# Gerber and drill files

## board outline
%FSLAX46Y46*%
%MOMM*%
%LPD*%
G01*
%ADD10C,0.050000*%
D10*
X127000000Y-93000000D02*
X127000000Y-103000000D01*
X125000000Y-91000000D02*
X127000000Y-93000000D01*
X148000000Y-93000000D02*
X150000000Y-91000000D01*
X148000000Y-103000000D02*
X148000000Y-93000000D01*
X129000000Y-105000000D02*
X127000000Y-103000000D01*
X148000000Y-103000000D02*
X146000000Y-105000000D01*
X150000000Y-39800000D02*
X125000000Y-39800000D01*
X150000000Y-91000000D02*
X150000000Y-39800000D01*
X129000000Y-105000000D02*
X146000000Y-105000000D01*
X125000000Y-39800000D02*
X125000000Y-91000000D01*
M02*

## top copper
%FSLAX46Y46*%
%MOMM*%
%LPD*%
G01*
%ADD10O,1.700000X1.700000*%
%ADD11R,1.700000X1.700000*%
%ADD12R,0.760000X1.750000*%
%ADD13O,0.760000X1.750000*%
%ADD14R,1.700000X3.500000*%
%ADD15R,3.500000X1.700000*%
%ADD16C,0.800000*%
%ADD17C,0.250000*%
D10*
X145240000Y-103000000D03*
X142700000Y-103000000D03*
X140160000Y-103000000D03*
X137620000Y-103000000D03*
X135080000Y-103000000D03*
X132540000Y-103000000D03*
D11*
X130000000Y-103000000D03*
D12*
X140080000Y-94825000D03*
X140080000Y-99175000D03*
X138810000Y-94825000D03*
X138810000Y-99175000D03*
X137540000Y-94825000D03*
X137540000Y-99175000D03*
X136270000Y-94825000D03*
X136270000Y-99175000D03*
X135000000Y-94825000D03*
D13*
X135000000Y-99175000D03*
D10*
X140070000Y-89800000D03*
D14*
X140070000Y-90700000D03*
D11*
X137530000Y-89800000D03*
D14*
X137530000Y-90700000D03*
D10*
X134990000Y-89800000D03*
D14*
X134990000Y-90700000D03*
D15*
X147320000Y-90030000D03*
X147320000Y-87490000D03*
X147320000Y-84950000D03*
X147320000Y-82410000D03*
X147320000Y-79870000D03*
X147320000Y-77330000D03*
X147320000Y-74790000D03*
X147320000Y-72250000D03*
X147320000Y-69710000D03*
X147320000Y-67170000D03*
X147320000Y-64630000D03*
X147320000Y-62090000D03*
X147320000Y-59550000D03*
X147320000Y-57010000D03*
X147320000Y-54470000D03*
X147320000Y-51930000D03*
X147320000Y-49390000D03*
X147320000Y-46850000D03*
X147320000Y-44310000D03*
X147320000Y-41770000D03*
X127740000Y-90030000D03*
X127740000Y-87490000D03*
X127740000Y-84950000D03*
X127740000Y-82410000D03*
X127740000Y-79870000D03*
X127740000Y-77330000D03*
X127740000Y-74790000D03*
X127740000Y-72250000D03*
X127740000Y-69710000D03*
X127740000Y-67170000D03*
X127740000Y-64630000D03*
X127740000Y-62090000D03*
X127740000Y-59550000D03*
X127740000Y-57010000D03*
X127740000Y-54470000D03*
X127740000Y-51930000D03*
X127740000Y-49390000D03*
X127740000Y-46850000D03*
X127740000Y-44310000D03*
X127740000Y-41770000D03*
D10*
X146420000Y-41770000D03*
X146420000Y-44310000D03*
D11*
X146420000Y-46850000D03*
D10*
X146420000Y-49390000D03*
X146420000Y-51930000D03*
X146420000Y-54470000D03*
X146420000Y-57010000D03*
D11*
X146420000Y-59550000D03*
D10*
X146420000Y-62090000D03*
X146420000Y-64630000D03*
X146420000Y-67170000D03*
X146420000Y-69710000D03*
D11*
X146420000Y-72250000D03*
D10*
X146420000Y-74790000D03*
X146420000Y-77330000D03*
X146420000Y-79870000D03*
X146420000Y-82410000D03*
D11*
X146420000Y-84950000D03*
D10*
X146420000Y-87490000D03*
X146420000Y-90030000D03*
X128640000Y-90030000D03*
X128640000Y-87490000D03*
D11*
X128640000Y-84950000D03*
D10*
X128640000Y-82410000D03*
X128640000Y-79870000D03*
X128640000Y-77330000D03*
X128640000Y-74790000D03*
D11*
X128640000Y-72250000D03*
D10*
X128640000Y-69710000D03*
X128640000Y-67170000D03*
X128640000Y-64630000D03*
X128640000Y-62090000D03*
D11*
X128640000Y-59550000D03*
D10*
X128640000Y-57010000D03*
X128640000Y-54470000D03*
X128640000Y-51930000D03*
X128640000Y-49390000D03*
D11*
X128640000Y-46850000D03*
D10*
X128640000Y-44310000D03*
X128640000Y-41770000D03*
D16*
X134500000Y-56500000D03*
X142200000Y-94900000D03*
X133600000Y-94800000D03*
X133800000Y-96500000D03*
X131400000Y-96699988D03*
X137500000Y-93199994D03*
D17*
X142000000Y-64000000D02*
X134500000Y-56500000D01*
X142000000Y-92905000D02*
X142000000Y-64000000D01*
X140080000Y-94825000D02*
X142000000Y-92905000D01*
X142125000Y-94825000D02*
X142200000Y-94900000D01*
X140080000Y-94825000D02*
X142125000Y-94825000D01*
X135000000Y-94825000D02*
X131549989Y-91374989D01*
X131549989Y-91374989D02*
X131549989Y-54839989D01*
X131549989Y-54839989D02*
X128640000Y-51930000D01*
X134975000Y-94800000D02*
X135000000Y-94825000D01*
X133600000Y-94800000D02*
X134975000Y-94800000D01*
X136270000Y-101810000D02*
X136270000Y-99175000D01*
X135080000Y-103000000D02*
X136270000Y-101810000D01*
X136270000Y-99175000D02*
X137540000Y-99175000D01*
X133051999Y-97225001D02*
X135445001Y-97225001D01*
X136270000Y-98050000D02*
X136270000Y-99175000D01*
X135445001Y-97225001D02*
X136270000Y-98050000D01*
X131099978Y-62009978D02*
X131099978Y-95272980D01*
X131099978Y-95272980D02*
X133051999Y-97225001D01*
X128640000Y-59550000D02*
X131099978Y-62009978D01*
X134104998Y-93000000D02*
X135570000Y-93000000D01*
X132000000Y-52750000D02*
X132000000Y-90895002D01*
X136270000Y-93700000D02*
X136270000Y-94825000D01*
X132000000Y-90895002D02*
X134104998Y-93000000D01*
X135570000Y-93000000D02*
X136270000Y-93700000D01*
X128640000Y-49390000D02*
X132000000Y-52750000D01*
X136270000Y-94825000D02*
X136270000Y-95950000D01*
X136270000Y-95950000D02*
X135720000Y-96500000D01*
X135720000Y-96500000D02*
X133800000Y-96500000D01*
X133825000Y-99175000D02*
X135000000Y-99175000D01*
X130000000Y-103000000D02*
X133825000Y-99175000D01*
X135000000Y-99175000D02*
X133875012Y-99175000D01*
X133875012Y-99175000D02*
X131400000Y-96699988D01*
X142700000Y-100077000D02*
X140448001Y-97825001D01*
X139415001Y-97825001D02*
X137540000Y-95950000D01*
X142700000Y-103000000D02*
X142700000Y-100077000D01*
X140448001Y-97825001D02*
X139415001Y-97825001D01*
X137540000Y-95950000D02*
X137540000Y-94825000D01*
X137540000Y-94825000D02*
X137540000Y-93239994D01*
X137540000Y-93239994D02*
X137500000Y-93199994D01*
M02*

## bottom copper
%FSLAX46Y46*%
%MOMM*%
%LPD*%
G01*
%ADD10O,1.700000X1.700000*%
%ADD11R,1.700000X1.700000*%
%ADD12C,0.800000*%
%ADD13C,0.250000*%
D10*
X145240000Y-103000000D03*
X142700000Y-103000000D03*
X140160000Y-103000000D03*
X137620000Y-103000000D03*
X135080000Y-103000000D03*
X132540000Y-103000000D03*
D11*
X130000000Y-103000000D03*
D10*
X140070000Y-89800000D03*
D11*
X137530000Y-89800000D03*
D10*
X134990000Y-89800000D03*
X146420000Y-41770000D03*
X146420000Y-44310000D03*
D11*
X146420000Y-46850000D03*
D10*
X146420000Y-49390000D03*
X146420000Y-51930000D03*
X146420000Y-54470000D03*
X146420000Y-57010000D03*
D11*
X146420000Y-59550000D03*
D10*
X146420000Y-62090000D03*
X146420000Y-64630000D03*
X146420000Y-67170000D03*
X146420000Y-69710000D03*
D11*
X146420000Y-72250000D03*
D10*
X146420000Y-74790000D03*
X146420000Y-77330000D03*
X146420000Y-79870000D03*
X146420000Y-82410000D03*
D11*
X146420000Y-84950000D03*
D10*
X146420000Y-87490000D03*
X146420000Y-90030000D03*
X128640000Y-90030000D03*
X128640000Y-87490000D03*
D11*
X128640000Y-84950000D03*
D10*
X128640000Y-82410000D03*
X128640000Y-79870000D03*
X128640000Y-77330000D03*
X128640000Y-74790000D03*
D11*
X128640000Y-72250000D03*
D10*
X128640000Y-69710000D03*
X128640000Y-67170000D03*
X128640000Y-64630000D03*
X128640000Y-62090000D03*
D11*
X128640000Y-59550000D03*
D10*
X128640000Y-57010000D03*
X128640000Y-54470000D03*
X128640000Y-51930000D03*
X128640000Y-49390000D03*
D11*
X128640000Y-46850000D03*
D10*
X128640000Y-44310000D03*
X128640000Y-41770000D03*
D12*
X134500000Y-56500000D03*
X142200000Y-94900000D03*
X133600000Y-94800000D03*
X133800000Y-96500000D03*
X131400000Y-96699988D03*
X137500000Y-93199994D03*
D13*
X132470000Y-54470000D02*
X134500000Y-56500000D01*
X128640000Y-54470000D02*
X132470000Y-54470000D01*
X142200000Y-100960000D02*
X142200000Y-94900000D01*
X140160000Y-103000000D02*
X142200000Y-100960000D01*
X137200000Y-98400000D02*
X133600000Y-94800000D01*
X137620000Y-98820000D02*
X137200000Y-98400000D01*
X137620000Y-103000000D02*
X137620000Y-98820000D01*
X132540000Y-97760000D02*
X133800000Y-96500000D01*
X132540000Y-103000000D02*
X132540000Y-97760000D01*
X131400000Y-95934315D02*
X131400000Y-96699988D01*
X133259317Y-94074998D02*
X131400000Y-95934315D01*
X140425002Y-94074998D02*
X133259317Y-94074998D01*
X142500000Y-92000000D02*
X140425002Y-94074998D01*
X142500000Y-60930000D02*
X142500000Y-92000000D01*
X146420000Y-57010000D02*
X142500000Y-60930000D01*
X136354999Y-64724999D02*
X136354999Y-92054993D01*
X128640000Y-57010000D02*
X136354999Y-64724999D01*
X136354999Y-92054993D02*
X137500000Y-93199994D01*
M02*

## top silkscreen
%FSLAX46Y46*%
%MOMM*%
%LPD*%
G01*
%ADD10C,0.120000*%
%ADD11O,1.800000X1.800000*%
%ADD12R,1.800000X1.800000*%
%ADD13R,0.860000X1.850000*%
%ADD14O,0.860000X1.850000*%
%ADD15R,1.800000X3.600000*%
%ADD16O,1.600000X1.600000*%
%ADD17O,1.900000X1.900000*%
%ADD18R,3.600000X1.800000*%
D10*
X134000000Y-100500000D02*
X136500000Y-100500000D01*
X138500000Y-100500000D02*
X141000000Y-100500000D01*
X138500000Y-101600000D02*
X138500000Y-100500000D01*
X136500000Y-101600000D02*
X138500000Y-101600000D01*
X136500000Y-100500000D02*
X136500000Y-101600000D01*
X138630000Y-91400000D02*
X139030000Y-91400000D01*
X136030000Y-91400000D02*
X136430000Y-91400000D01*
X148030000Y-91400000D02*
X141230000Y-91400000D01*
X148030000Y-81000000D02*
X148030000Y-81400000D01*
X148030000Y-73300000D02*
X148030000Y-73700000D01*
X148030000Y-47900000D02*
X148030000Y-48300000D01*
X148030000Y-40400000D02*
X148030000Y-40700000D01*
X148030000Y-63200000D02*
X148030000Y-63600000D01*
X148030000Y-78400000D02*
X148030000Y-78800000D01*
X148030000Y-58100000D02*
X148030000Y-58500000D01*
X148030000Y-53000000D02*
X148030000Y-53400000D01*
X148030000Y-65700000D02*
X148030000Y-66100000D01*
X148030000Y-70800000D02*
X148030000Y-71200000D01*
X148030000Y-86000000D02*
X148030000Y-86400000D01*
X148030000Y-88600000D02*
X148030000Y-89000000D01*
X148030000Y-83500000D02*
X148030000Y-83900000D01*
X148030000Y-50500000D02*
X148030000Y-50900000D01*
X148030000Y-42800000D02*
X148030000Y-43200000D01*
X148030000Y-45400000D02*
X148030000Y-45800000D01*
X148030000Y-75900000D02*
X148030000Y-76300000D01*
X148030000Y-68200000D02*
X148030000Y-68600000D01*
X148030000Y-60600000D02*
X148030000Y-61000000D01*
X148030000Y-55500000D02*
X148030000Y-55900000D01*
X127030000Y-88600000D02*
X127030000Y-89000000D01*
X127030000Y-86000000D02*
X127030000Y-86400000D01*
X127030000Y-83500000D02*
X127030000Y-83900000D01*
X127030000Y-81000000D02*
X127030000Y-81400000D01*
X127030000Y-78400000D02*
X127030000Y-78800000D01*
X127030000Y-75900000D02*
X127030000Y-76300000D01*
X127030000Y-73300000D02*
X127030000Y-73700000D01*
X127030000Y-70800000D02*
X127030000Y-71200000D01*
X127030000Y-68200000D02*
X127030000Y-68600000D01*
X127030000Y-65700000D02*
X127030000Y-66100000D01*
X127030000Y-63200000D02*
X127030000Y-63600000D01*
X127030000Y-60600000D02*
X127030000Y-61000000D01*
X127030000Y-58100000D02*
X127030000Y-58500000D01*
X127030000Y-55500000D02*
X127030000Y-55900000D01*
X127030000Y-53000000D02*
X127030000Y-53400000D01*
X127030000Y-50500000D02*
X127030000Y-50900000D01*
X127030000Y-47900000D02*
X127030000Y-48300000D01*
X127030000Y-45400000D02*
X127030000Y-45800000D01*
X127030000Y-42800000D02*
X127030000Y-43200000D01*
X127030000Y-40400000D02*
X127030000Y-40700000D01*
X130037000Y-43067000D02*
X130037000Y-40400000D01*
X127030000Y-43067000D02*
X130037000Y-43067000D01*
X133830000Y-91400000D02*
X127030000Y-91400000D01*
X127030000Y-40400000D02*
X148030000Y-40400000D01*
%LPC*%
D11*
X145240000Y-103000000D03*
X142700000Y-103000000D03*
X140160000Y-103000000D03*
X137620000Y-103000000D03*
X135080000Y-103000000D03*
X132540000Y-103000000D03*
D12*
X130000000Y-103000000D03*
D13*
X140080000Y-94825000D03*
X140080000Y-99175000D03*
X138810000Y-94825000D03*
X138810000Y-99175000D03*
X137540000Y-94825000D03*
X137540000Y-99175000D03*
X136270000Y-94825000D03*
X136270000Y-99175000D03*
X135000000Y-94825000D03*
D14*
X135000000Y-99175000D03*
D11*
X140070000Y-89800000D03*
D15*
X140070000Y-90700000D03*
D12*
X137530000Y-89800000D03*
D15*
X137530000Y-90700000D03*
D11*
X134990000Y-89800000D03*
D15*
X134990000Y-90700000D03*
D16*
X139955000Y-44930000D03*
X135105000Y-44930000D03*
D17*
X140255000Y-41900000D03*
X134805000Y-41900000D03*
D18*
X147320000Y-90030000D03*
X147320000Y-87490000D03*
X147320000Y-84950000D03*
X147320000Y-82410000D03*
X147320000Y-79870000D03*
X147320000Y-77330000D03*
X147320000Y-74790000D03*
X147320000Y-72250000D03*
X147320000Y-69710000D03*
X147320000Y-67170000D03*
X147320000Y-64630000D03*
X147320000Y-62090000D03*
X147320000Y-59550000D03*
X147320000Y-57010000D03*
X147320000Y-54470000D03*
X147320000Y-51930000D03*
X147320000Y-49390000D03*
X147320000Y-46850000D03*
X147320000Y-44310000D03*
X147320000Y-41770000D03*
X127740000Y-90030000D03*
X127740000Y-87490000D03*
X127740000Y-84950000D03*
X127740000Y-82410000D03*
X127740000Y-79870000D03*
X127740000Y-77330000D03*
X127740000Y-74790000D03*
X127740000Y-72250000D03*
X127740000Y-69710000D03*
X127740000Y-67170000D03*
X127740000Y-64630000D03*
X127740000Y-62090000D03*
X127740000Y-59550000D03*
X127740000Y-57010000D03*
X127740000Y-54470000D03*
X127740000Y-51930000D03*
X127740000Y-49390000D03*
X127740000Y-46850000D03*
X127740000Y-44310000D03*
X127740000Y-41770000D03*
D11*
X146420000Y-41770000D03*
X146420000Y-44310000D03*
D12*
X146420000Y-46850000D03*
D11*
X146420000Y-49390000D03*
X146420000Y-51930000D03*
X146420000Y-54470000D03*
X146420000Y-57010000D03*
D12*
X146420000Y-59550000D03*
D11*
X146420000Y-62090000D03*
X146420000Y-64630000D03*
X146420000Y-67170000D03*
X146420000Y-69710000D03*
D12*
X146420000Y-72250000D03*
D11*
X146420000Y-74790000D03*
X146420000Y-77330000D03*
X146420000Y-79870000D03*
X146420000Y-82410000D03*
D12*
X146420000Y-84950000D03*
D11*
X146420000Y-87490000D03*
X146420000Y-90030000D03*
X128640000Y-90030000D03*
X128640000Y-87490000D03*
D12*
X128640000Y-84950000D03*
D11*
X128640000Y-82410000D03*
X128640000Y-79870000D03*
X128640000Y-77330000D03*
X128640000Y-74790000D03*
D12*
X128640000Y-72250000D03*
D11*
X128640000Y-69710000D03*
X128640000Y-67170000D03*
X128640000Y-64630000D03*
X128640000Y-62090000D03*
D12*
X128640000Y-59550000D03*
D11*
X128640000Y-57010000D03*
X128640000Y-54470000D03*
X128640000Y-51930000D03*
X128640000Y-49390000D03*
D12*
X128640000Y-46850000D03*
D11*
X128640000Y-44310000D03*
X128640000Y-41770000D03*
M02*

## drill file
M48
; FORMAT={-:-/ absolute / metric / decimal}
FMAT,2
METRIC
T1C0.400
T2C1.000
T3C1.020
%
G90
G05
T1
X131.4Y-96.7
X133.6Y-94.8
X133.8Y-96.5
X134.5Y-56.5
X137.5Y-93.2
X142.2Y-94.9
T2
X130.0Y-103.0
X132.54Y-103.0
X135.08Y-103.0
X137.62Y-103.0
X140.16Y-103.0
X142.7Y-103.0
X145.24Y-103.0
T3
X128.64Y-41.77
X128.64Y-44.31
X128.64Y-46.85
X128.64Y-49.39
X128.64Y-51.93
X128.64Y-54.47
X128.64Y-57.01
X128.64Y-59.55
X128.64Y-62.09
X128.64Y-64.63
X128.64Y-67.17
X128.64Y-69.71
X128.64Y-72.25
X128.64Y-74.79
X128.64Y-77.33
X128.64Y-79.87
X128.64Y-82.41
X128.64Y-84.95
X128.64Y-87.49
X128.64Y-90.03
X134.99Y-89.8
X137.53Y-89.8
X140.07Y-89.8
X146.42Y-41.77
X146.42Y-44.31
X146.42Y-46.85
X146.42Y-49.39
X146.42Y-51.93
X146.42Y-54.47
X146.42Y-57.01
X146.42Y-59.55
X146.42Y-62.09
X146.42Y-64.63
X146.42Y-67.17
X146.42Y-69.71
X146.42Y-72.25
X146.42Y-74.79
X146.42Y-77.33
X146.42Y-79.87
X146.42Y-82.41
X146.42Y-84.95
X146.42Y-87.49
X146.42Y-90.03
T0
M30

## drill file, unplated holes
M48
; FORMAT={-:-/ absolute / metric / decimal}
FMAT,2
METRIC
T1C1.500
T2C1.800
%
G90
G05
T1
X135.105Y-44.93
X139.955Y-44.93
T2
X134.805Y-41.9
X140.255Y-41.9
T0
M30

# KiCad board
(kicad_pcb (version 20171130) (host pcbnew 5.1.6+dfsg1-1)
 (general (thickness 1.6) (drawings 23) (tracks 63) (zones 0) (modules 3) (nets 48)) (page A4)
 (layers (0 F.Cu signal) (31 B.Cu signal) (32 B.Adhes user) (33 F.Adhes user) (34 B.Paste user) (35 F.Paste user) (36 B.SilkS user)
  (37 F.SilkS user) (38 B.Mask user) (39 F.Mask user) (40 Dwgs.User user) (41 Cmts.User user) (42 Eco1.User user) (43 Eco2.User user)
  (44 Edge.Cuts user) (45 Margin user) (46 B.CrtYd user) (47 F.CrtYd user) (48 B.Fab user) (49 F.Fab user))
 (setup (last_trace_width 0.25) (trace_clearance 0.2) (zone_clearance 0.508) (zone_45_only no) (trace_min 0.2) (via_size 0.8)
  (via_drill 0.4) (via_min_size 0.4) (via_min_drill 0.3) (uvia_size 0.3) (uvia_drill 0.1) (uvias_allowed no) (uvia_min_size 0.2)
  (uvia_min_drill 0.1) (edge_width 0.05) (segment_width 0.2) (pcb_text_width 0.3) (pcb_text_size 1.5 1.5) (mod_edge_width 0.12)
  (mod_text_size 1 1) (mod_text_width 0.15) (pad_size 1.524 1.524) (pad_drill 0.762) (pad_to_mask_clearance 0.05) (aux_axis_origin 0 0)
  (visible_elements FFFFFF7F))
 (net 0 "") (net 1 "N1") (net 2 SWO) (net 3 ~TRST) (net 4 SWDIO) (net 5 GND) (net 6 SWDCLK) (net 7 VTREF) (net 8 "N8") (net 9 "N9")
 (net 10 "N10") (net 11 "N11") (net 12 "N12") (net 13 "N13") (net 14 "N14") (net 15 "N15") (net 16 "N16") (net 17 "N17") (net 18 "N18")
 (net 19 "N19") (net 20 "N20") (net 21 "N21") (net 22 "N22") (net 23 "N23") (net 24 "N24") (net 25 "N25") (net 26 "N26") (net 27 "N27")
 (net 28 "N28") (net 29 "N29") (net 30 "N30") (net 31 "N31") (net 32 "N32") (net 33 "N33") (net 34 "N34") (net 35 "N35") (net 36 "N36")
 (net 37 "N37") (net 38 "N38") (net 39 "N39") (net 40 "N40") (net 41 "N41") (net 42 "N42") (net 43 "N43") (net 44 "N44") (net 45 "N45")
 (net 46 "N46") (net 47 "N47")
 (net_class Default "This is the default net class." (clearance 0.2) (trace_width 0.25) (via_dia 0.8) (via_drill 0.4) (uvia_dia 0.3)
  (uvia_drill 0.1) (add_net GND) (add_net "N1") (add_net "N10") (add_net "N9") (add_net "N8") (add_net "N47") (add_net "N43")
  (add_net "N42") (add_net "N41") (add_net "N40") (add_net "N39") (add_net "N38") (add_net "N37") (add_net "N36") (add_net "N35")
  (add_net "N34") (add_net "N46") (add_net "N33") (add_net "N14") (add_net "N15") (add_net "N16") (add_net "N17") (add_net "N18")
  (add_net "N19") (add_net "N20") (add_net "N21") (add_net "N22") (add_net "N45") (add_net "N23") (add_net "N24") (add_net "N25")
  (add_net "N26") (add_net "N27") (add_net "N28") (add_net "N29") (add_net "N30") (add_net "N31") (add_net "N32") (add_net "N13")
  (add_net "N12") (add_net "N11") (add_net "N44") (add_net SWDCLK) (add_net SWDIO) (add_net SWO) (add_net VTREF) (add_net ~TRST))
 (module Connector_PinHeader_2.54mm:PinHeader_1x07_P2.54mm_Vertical (layer B.Cu) (at 130 103 270)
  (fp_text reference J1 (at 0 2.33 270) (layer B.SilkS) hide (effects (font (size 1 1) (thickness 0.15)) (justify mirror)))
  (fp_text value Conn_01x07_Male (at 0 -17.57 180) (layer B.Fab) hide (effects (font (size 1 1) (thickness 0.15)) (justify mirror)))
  (pad 7 thru_hole oval (at 0 -15.24 270) (size 1.7 1.7) (drill 1) (layers *.Cu *.Mask) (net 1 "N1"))
  (pad 6 thru_hole oval (at 0 -12.7 270) (size 1.7 1.7) (drill 1) (layers *.Cu *.Mask) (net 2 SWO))
  (pad 5 thru_hole oval (at 0 -10.16 270) (size 1.7 1.7) (drill 1) (layers *.Cu *.Mask) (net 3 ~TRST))
  (pad 4 thru_hole oval (at 0 -7.62 270) (size 1.7 1.7) (drill 1) (layers *.Cu *.Mask) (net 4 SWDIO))
  (pad 3 thru_hole oval (at 0 -5.08 270) (size 1.7 1.7) (drill 1) (layers *.Cu *.Mask) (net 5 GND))
  (pad 2 thru_hole oval (at 0 -2.54 270) (size 1.7 1.7) (drill 1) (layers *.Cu *.Mask) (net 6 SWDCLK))
  (pad 1 thru_hole rect (at 0 0 270) (size 1.7 1.7) (drill 1) (layers *.Cu *.Mask) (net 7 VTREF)))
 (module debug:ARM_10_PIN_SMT (layer F.Cu) (at 137.5 97)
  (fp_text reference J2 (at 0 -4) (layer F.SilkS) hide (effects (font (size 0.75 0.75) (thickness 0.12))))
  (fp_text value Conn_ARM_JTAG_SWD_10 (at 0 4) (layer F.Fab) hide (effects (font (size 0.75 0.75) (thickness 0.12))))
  (pad 10 smd rect (at 2.58 -2.175) (size 0.76 1.75) (layers F.Cu F.Paste F.Mask) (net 3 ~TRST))
  (pad 9 smd rect (at 2.58 2.175) (size 0.76 1.75) (layers F.Cu F.Paste F.Mask) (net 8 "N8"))
  (pad 8 smd rect (at 1.31 -2.175) (size 0.76 1.75) (layers F.Cu F.Paste F.Mask) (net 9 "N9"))
  (pad 7 smd rect (at 1.31 2.175) (size 0.76 1.75) (layers F.Cu F.Paste F.Mask) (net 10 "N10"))
  (pad 6 smd rect (at 0.04 -2.175) (size 0.76 1.75) (layers F.Cu F.Paste F.Mask) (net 2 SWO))
  (pad 5 smd rect (at 0.04 2.175) (size 0.76 1.75) (layers F.Cu F.Paste F.Mask) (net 5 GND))
  (pad 4 smd rect (at -1.23 -2.175) (size 0.76 1.75) (layers F.Cu F.Paste F.Mask) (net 6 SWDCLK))
  (pad 3 smd rect (at -1.23 2.175) (size 0.76 1.75) (layers F.Cu F.Paste F.Mask) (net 5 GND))
  (pad 2 smd rect (at -2.5 -2.175) (size 0.76 1.75) (layers F.Cu F.Paste F.Mask) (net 4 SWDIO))
  (pad 1 smd oval (at -2.5 2.175) (size 0.76 1.75) (layers F.Cu F.Paste F.Mask) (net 7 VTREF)))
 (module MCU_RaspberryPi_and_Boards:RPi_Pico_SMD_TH (layer F.Cu) (at 137.53 65.9)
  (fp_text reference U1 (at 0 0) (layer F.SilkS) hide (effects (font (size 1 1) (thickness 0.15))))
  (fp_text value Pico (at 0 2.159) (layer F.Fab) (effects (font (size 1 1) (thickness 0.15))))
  (fp_line (start 1.1 25.5) (end 1.5 25.5) (layer F.SilkS) (width 0.12))
  (fp_line (start -1.5 25.5) (end -1.1 25.5) (layer F.SilkS) (width 0.12))
  (fp_line (start 10.5 25.5) (end 3.7 25.5) (layer F.SilkS) (width 0.12))
  (fp_line (start 10.5 15.1) (end 10.5 15.5) (layer F.SilkS) (width 0.12))
  (fp_line (start 10.5 7.4) (end 10.5 7.8) (layer F.SilkS) (width 0.12))
  (fp_line (start 10.5 -18) (end 10.5 -17.6) (layer F.SilkS) (width 0.12))
  (fp_line (start 10.5 -25.5) (end 10.5 -25.2) (layer F.SilkS) (width 0.12))
  (fp_line (start 10.5 -2.7) (end 10.5 -2.3) (layer F.SilkS) (width 0.12))
  (fp_line (start 10.5 12.5) (end 10.5 12.9) (layer F.SilkS) (width 0.12))
  (fp_line (start 10.5 -7.8) (end 10.5 -7.4) (layer F.SilkS) (width 0.12))
  (fp_line (start 10.5 -12.9) (end 10.5 -12.5) (layer F.SilkS) (width 0.12))
  (fp_line (start 10.5 -0.2) (end 10.5 0.2) (layer F.SilkS) (width 0.12))
  (fp_line (start 10.5 4.9) (end 10.5 5.3) (layer F.SilkS) (width 0.12))
  (fp_line (start 10.5 20.1) (end 10.5 20.5) (layer F.SilkS) (width 0.12))
  (fp_line (start 10.5 22.7) (end 10.5 23.1) (layer F.SilkS) (width 0.12))
  (fp_line (start 10.5 17.6) (end 10.5 18) (layer F.SilkS) (width 0.12))
  (fp_line (start 10.5 -15.4) (end 10.5 -15) (layer F.SilkS) (width 0.12))
  (fp_line (start 10.5 -23.1) (end 10.5 -22.7) (layer F.SilkS) (width 0.12))
  (fp_line (start 10.5 -20.5) (end 10.5 -20.1) (layer F.SilkS) (width 0.12))
  (fp_line (start 10.5 10) (end 10.5 10.4) (layer F.SilkS) (width 0.12))
  (fp_line (start 10.5 2.3) (end 10.5 2.7) (layer F.SilkS) (width 0.12))
  (fp_line (start 10.5 -5.3) (end 10.5 -4.9) (layer F.SilkS) (width 0.12))
  (fp_line (start 10.5 -10.4) (end 10.5 -10) (layer F.SilkS) (width 0.12))
  (fp_line (start -10.5 22.7) (end -10.5 23.1) (layer F.SilkS) (width 0.12))
  (fp_line (start -10.5 20.1) (end -10.5 20.5) (layer F.SilkS) (width 0.12))
  (fp_line (start -10.5 17.6) (end -10.5 18) (layer F.SilkS) (width 0.12))
  (fp_line (start -10.5 15.1) (end -10.5 15.5) (layer F.SilkS) (width 0.12))
  (fp_line (start -10.5 12.5) (end -10.5 12.9) (layer F.SilkS) (width 0.12))
  (fp_line (start -10.5 10) (end -10.5 10.4) (layer F.SilkS) (width 0.12))
  (fp_line (start -10.5 7.4) (end -10.5 7.8) (layer F.SilkS) (width 0.12))
  (fp_line (start -10.5 4.9) (end -10.5 5.3) (layer F.SilkS) (width 0.12))
  (fp_line (start -10.5 2.3) (end -10.5 2.7) (layer F.SilkS) (width 0.12))
  (fp_line (start -10.5 -0.2) (end -10.5 0.2) (layer F.SilkS) (width 0.12))
  (fp_line (start -10.5 -2.7) (end -10.5 -2.3) (layer F.SilkS) (width 0.12))
  (fp_line (start -10.5 -5.3) (end -10.5 -4.9) (layer F.SilkS) (width 0.12))
  (fp_line (start -10.5 -7.8) (end -10.5 -7.4) (layer F.SilkS) (width 0.12))
  (fp_line (start -10.5 -10.4) (end -10.5 -10) (layer F.SilkS) (width 0.12))
  (fp_line (start -10.5 -12.9) (end -10.5 -12.5) (layer F.SilkS) (width 0.12))
  (fp_line (start -10.5 -15.4) (end -10.5 -15) (layer F.SilkS) (width 0.12))
  (fp_line (start -10.5 -18) (end -10.5 -17.6) (layer F.SilkS) (width 0.12))
  (fp_line (start -10.5 -20.5) (end -10.5 -20.1) (layer F.SilkS) (width 0.12))
  (fp_line (start -10.5 -23.1) (end -10.5 -22.7) (layer F.SilkS) (width 0.12))
  (fp_line (start -10.5 -25.5) (end -10.5 -25.2) (layer F.SilkS) (width 0.12))
  (fp_line (start -7.493 -22.833) (end -7.493 -25.5) (layer F.SilkS) (width 0.12))
  (fp_line (start -10.5 -22.833) (end -7.493 -22.833) (layer F.SilkS) (width 0.12))
  (fp_line (start -3.7 25.5) (end -10.5 25.5) (layer F.SilkS) (width 0.12))
  (fp_line (start -10.5 -25.5) (end 10.5 -25.5) (layer F.SilkS) (width 0.12))
  (pad 43 thru_hole oval (at 2.54 23.9) (size 1.7 1.7) (drill 1.02) (layers *.Cu *.Mask) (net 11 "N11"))
  (pad 43 smd rect (at 2.54 23.9 90) (size 3.5 1.7) (drill (offset -0.9 0)) (layers F.Cu F.Mask) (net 11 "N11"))
  (pad 42 thru_hole rect (at 0 23.9) (size 1.7 1.7) (drill 1.02) (layers *.Cu *.Mask) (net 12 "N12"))
  (pad 42 smd rect (at 0 23.9 90) (size 3.5 1.7) (drill (offset -0.9 0)) (layers F.Cu F.Mask) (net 12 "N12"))
  (pad 41 thru_hole oval (at -2.54 23.9) (size 1.7 1.7) (drill 1.02) (layers *.Cu *.Mask) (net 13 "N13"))
  (pad 41 smd rect (at -2.54 23.9 90) (size 3.5 1.7) (drill (offset -0.9 0)) (layers F.Cu F.Mask) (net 13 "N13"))
  (pad "" np_thru_hole oval (at 2.425 -20.97) (size 1.5 1.5) (drill 1.5) (layers *.Cu *.Mask))
  (pad "" np_thru_hole oval (at -2.425 -20.97) (size 1.5 1.5) (drill 1.5) (layers *.Cu *.Mask))
  (pad "" np_thru_hole oval (at 2.725 -24) (size 1.8 1.8) (drill 1.8) (layers *.Cu *.Mask))
  (pad "" np_thru_hole oval (at -2.725 -24) (size 1.8 1.8) (drill 1.8) (layers *.Cu *.Mask))
  (pad 21 smd rect (at 8.89 24.13) (size 3.5 1.7) (drill (offset 0.9 0)) (layers F.Cu F.Mask) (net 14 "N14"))
  (pad 22 smd rect (at 8.89 21.59) (size 3.5 1.7) (drill (offset 0.9 0)) (layers F.Cu F.Mask) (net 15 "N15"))
  (pad 23 smd rect (at 8.89 19.05) (size 3.5 1.7) (drill (offset 0.9 0)) (layers F.Cu F.Mask) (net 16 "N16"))
  (pad 24 smd rect (at 8.89 16.51) (size 3.5 1.7) (drill (offset 0.9 0)) (layers F.Cu F.Mask) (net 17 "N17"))
  (pad 25 smd rect (at 8.89 13.97) (size 3.5 1.7) (drill (offset 0.9 0)) (layers F.Cu F.Mask) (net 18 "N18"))
  (pad 26 smd rect (at 8.89 11.43) (size 3.5 1.7) (drill (offset 0.9 0)) (layers F.Cu F.Mask) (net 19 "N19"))
  (pad 27 smd rect (at 8.89 8.89) (size 3.5 1.7) (drill (offset 0.9 0)) (layers F.Cu F.Mask) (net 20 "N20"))
  (pad 28 smd rect (at 8.89 6.35) (size 3.5 1.7) (drill (offset 0.9 0)) (layers F.Cu F.Mask) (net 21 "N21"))
  (pad 29 smd rect (at 8.89 3.81) (size 3.5 1.7) (drill (offset 0.9 0)) (layers F.Cu F.Mask) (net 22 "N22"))
  (pad 30 smd rect (at 8.89 1.27) (size 3.5 1.7) (drill (offset 0.9 0)) (layers F.Cu F.Mask) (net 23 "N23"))
  (pad 31 smd rect (at 8.89 -1.27) (size 3.5 1.7) (drill (offset 0.9 0)) (layers F.Cu F.Mask) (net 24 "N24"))
  (pad 32 smd rect (at 8.89 -3.81) (size 3.5 1.7) (drill (offset 0.9 0)) (layers F.Cu F.Mask) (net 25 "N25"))
  (pad 33 smd rect (at 8.89 -6.35) (size 3.5 1.7) (drill (offset 0.9 0)) (layers F.Cu F.Mask) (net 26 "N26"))
  (pad 34 smd rect (at 8.89 -8.89) (size 3.5 1.7) (drill (offset 0.9 0)) (layers F.Cu F.Mask) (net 7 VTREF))
  (pad 35 smd rect (at 8.89 -11.43) (size 3.5 1.7) (drill (offset 0.9 0)) (layers F.Cu F.Mask) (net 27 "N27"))
  (pad 36 smd rect (at 8.89 -13.97) (size 3.5 1.7) (drill (offset 0.9 0)) (layers F.Cu F.Mask) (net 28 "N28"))
  (pad 37 smd rect (at 8.89 -16.51) (size 3.5 1.7) (drill (offset 0.9 0)) (layers F.Cu F.Mask) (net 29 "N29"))
  (pad 38 smd rect (at 8.89 -19.05) (size 3.5 1.7) (drill (offset 0.9 0)) (layers F.Cu F.Mask) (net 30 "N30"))
  (pad 39 smd rect (at 8.89 -21.59) (size 3.5 1.7) (drill (offset 0.9 0)) (layers F.Cu F.Mask) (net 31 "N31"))
  (pad 40 smd rect (at 8.89 -24.13) (size 3.5 1.7) (drill (offset 0.9 0)) (layers F.Cu F.Mask) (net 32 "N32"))
  (pad 20 smd rect (at -8.89 24.13) (size 3.5 1.7) (drill (offset -0.9 0)) (layers F.Cu F.Mask) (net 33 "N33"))
  (pad 19 smd rect (at -8.89 21.59) (size 3.5 1.7) (drill (offset -0.9 0)) (layers F.Cu F.Mask) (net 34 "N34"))
  (pad 18 smd rect (at -8.89 19.05) (size 3.5 1.7) (drill (offset -0.9 0)) (layers F.Cu F.Mask) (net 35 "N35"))
  (pad 17 smd rect (at -8.89 16.51) (size 3.5 1.7) (drill (offset -0.9 0)) (layers F.Cu F.Mask) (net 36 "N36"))
  (pad 16 smd rect (at -8.89 13.97) (size 3.5 1.7) (drill (offset -0.9 0)) (layers F.Cu F.Mask) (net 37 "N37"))
  (pad 15 smd rect (at -8.89 11.43) (size 3.5 1.7) (drill (offset -0.9 0)) (layers F.Cu F.Mask) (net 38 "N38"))
  (pad 14 smd rect (at -8.89 8.89) (size 3.5 1.7) (drill (offset -0.9 0)) (layers F.Cu F.Mask) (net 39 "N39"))
  (pad 13 smd rect (at -8.89 6.35) (size 3.5 1.7) (drill (offset -0.9 0)) (layers F.Cu F.Mask) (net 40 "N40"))
  (pad 12 smd rect (at -8.89 3.81) (size 3.5 1.7) (drill (offset -0.9 0)) (layers F.Cu F.Mask) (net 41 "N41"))
  (pad 11 smd rect (at -8.89 1.27) (size 3.5 1.7) (drill (offset -0.9 0)) (layers F.Cu F.Mask) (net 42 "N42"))
  (pad 10 smd rect (at -8.89 -1.27) (size 3.5 1.7) (drill (offset -0.9 0)) (layers F.Cu F.Mask) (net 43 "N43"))
  (pad 9 smd rect (at -8.89 -3.81) (size 3.5 1.7) (drill (offset -0.9 0)) (layers F.Cu F.Mask) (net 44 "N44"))
  (pad 8 smd rect (at -8.89 -6.35) (size 3.5 1.7) (drill (offset -0.9 0)) (layers F.Cu F.Mask) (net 5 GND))
  (pad 7 smd rect (at -8.89 -8.89) (size 3.5 1.7) (drill (offset -0.9 0)) (layers F.Cu F.Mask) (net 2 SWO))
  (pad 6 smd rect (at -8.89 -11.43) (size 3.5 1.7) (drill (offset -0.9 0)) (layers F.Cu F.Mask) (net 3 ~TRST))
  (pad 5 smd rect (at -8.89 -13.97) (size 3.5 1.7) (drill (offset -0.9 0)) (layers F.Cu F.Mask) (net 4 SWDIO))
  (pad 4 smd rect (at -8.89 -16.51) (size 3.5 1.7) (drill (offset -0.9 0)) (layers F.Cu F.Mask) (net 6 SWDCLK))
  (pad 3 smd rect (at -8.89 -19.05) (size 3.5 1.7) (drill (offset -0.9 0)) (layers F.Cu F.Mask) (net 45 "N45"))
  (pad 2 smd rect (at -8.89 -21.59) (size 3.5 1.7) (drill (offset -0.9 0)) (layers F.Cu F.Mask) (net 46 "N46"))
  (pad 1 smd rect (at -8.89 -24.13) (size 3.5 1.7) (drill (offset -0.9 0)) (layers F.Cu F.Mask) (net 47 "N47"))
  (pad 40 thru_hole oval (at 8.89 -24.13) (size 1.7 1.7) (drill 1.02) (layers *.Cu *.Mask) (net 32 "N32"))
  (pad 39 thru_hole oval (at 8.89 -21.59) (size 1.7 1.7) (drill 1.02) (layers *.Cu *.Mask) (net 31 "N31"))
  (pad 38 thru_hole rect (at 8.89 -19.05) (size 1.7 1.7) (drill 1.02) (layers *.Cu *.Mask) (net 30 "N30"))
  (pad 37 thru_hole oval (at 8.89 -16.51) (size 1.7 1.7) (drill 1.02) (layers *.Cu *.Mask) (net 29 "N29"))
  (pad 36 thru_hole oval (at 8.89 -13.97) (size 1.7 1.7) (drill 1.02) (layers *.Cu *.Mask) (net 28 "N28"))
  (pad 35 thru_hole oval (at 8.89 -11.43) (size 1.7 1.7) (drill 1.02) (layers *.Cu *.Mask) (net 27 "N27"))
  (pad 34 thru_hole oval (at 8.89 -8.89) (size 1.7 1.7) (drill 1.02) (layers *.Cu *.Mask) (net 7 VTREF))
  (pad 33 thru_hole rect (at 8.89 -6.35) (size 1.7 1.7) (drill 1.02) (layers *.Cu *.Mask) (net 26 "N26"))
  (pad 32 thru_hole oval (at 8.89 -3.81) (size 1.7 1.7) (drill 1.02) (layers *.Cu *.Mask) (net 25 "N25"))
  (pad 31 thru_hole oval (at 8.89 -1.27) (size 1.7 1.7) (drill 1.02) (layers *.Cu *.Mask) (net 24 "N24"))
  (pad 30 thru_hole oval (at 8.89 1.27) (size 1.7 1.7) (drill 1.02) (layers *.Cu *.Mask) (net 23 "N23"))
  (pad 29 thru_hole oval (at 8.89 3.81) (size 1.7 1.7) (drill 1.02) (layers *.Cu *.Mask) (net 22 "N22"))
  (pad 28 thru_hole rect (at 8.89 6.35) (size 1.7 1.7) (drill 1.02) (layers *.Cu *.Mask) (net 21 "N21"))
  (pad 27 thru_hole oval (at 8.89 8.89) (size 1.7 1.7) (drill 1.02) (layers *.Cu *.Mask) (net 20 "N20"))
  (pad 26 thru_hole oval (at 8.89 11.43) (size 1.7 1.7) (drill 1.02) (layers *.Cu *.Mask) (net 19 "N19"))
  (pad 25 thru_hole oval (at 8.89 13.97) (size 1.7 1.7) (drill 1.02) (layers *.Cu *.Mask) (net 18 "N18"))
  (pad 24 thru_hole oval (at 8.89 16.51) (size 1.7 1.7) (drill 1.02) (layers *.Cu *.Mask) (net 17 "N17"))
  (pad 23 thru_hole rect (at 8.89 19.05) (size 1.7 1.7) (drill 1.02) (layers *.Cu *.Mask) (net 16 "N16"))
  (pad 22 thru_hole oval (at 8.89 21.59) (size 1.7 1.7) (drill 1.02) (layers *.Cu *.Mask) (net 15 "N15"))
  (pad 21 thru_hole oval (at 8.89 24.13) (size 1.7 1.7) (drill 1.02) (layers *.Cu *.Mask) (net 14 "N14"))
  (pad 20 thru_hole oval (at -8.89 24.13) (size 1.7 1.7) (drill 1.02) (layers *.Cu *.Mask) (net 33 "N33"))
  (pad 19 thru_hole oval (at -8.89 21.59) (size 1.7 1.7) (drill 1.02) (layers *.Cu *.Mask) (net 34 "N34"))
  (pad 18 thru_hole rect (at -8.89 19.05) (size 1.7 1.7) (drill 1.02) (layers *.Cu *.Mask) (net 35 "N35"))
  (pad 17 thru_hole oval (at -8.89 16.51) (size 1.7 1.7) (drill 1.02) (layers *.Cu *.Mask) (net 36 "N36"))
  (pad 16 thru_hole oval (at -8.89 13.97) (size 1.7 1.7) (drill 1.02) (layers *.Cu *.Mask) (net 37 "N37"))
  (pad 15 thru_hole oval (at -8.89 11.43) (size 1.7 1.7) (drill 1.02) (layers *.Cu *.Mask) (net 38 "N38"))
  (pad 14 thru_hole oval (at -8.89 8.89) (size 1.7 1.7) (drill 1.02) (layers *.Cu *.Mask) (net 39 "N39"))
  (pad 13 thru_hole rect (at -8.89 6.35) (size 1.7 1.7) (drill 1.02) (layers *.Cu *.Mask) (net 40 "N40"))
  (pad 12 thru_hole oval (at -8.89 3.81) (size 1.7 1.7) (drill 1.02) (layers *.Cu *.Mask) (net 41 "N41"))
  (pad 11 thru_hole oval (at -8.89 1.27) (size 1.7 1.7) (drill 1.02) (layers *.Cu *.Mask) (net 42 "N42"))
  (pad 10 thru_hole oval (at -8.89 -1.27) (size 1.7 1.7) (drill 1.02) (layers *.Cu *.Mask) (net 43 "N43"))
  (pad 9 thru_hole oval (at -8.89 -3.81) (size 1.7 1.7) (drill 1.02) (layers *.Cu *.Mask) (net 44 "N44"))
  (pad 8 thru_hole rect (at -8.89 -6.35) (size 1.7 1.7) (drill 1.02) (layers *.Cu *.Mask) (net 5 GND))
  (pad 7 thru_hole oval (at -8.89 -8.89) (size 1.7 1.7) (drill 1.02) (layers *.Cu *.Mask) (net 2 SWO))
  (pad 6 thru_hole oval (at -8.89 -11.43) (size 1.7 1.7) (drill 1.02) (layers *.Cu *.Mask) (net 3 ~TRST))
  (pad 5 thru_hole oval (at -8.89 -13.97) (size 1.7 1.7) (drill 1.02) (layers *.Cu *.Mask) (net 4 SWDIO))
  (pad 4 thru_hole oval (at -8.89 -16.51) (size 1.7 1.7) (drill 1.02) (layers *.Cu *.Mask) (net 6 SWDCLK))
  (pad 3 thru_hole rect (at -8.89 -19.05) (size 1.7 1.7) (drill 1.02) (layers *.Cu *.Mask) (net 45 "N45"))
  (pad 2 thru_hole oval (at -8.89 -21.59) (size 1.7 1.7) (drill 1.02) (layers *.Cu *.Mask) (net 46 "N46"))
  (pad 1 thru_hole oval (at -8.89 -24.13) (size 1.7 1.7) (drill 1.02) (layers *.Cu *.Mask) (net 47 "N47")))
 (gr_line (start 127 93) (end 127 103) (layer Edge.Cuts) (width 0.05))
 (gr_line (start 125 91) (end 127 93) (layer Edge.Cuts) (width 0.05))
 (gr_line (start 148 93) (end 150 91) (layer Edge.Cuts) (width 0.05))
 (gr_line (start 148 103) (end 148 93) (layer Edge.Cuts) (width 0.05))
 (gr_line (start 134 100.5) (end 136.5 100.5) (layer F.SilkS) (width 0.12))
 (gr_line (start 138.5 100.5) (end 141 100.5) (layer F.SilkS) (width 0.12))
 (gr_line (start 138.5 101.6) (end 138.5 100.5) (layer F.SilkS) (width 0.12))
 (gr_line (start 136.5 101.6) (end 138.5 101.6) (layer F.SilkS) (width 0.12))
 (gr_line (start 136.5 100.5) (end 136.5 101.6) (layer F.SilkS) (width 0.12))
 (gr_line (start 129 105) (end 127 103) (layer Edge.Cuts) (width 0.05))
 (gr_line (start 148 103) (end 146 105) (layer Edge.Cuts) (width 0.05))
 (gr_line (start 150 39.8) (end 125 39.8) (layer Edge.Cuts) (width 0.05))
 (gr_line (start 150 91) (end 150 39.8) (layer Edge.Cuts) (width 0.05))
 (gr_line (start 129 105) (end 146 105) (layer Edge.Cuts) (width 0.05))
 (gr_line (start 125 39.8) (end 125 91) (layer Edge.Cuts) (width 0.05))
 (segment (start 132.47 54.47) (end 134.5 56.5) (width 0.25) (layer B.Cu) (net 3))
 (segment (start 128.64 54.47) (end 132.47 54.47) (width 0.25) (layer B.Cu) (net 3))
 (segment (start 142 64) (end 134.5 56.5) (width 0.25) (layer F.Cu) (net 3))
 (segment (start 142 92.905) (end 142 64) (width 0.25) (layer F.Cu) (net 3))
 (segment (start 140.08 94.825) (end 142 92.905) (width 0.25) (layer F.Cu) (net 3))
 (via (at 134.5 56.5) (size 0.8) (drill 0.4) (layers F.Cu B.Cu) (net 3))
 (segment (start 142.125 94.825) (end 142.2 94.9) (width 0.25) (layer F.Cu) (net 3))
 (via (at 142.2 94.9) (size 0.8) (drill 0.4) (layers F.Cu B.Cu) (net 3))
 (segment (start 140.08 94.825) (end 142.125 94.825) (width 0.25) (layer F.Cu) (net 3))
 (segment (start 142.2 100.96) (end 142.2 94.9) (width 0.25) (layer B.Cu) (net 3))
 (segment (start 140.16 103) (end 142.2 100.96) (width 0.25) (layer B.Cu) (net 3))
 (segment (start 135 94.825) (end 131.549989 91.374989) (width 0.25) (layer F.Cu) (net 4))
 (segment (start 131.549989 91.374989) (end 131.549989 54.839989) (width 0.25) (layer F.Cu) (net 4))
 (segment (start 131.549989 54.839989) (end 128.64 51.93) (width 0.25) (layer F.Cu) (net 4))
 (via (at 133.6 94.8) (size 0.8) (drill 0.4) (layers F.Cu B.Cu) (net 4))
 (segment (start 134.975 94.8) (end 135 94.825) (width 0.25) (layer F.Cu) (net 4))
 (segment (start 133.6 94.8) (end 134.975 94.8) (width 0.25) (layer F.Cu) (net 4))
 (segment (start 137.2 98.4) (end 133.6 94.8) (width 0.25) (layer B.Cu) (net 4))
 (segment (start 137.62 98.82) (end 137.2 98.4) (width 0.25) (layer B.Cu) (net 4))
 (segment (start 137.62 103) (end 137.62 98.82) (width 0.25) (layer B.Cu) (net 4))
 (segment (start 136.27 101.81) (end 136.27 99.175) (width 0.25) (layer F.Cu) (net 5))
 (segment (start 135.08 103) (end 136.27 101.81) (width 0.25) (layer F.Cu) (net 5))
 (segment (start 136.27 99.175) (end 137.54 99.175) (width 0.25) (layer F.Cu) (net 5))
 (segment (start 133.051999 97.225001) (end 135.445001 97.225001) (width 0.25) (layer F.Cu) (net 5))
 (segment (start 136.27 98.05) (end 136.27 99.175) (width 0.25) (layer F.Cu) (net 5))
 (segment (start 135.445001 97.225001) (end 136.27 98.05) (width 0.25) (layer F.Cu) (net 5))
 (segment (start 131.099978 62.009978) (end 131.099978 95.27298) (width 0.25) (layer F.Cu) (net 5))
 (segment (start 131.099978 95.27298) (end 133.051999 97.225001) (width 0.25) (layer F.Cu) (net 5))
 (segment (start 128.64 59.55) (end 131.099978 62.009978) (width 0.25) (layer F.Cu) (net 5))
 (segment (start 134.104998 93) (end 135.57 93) (width 0.25) (layer F.Cu) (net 6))
 (segment (start 132 52.75) (end 132 90.895002) (width 0.25) (layer F.Cu) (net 6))
 (segment (start 136.27 93.7) (end 136.27 94.825) (width 0.25) (layer F.Cu) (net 6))
 (segment (start 132 90.895002) (end 134.104998 93) (width 0.25) (layer F.Cu) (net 6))
 (segment (start 135.57 93) (end 136.27 93.7) (width 0.25) (layer F.Cu) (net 6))
 (segment (start 128.64 49.39) (end 132 52.75) (width 0.25) (layer F.Cu) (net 6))
 (via (at 133.8 96.5) (size 0.8) (drill 0.4) (layers F.Cu B.Cu) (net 6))
 (segment (start 132.54 97.76) (end 133.8 96.5) (width 0.25) (layer B.Cu) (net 6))
 (segment (start 136.27 94.825) (end 136.27 95.95) (width 0.25) (layer F.Cu) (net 6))
 (segment (start 136.27 95.95) (end 135.72 96.5) (width 0.25) (layer F.Cu) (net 6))
 (segment (start 135.72 96.5) (end 133.8 96.5) (width 0.25) (layer F.Cu) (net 6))
 (segment (start 132.54 103) (end 132.54 97.76) (width 0.25) (layer B.Cu) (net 6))
 (segment (start 133.825 99.175) (end 135 99.175) (width 0.25) (layer F.Cu) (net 7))
 (segment (start 130 103) (end 133.825 99.175) (width 0.25) (layer F.Cu) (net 7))
 (via (at 131.4 96.699988) (size 0.8) (drill 0.4) (layers F.Cu B.Cu) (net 7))
 (segment (start 135 99.175) (end 133.875012 99.175) (width 0.25) (layer F.Cu) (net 7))
 (segment (start 133.875012 99.175) (end 131.4 96.699988) (width 0.25) (layer F.Cu) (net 7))
 (segment (start 131.4 95.934315) (end 131.4 96.699988) (width 0.25) (layer B.Cu) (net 7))
 (segment (start 133.259317 94.074998) (end 131.4 95.934315) (width 0.25) (layer B.Cu) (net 7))
 (segment (start 140.425002 94.074998) (end 133.259317 94.074998) (width 0.25) (layer B.Cu) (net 7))
 (segment (start 142.5 92) (end 140.425002 94.074998) (width 0.25) (layer B.Cu) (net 7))
 (segment (start 142.5 60.93) (end 142.5 92) (width 0.25) (layer B.Cu) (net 7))
 (segment (start 146.42 57.01) (end 142.5 60.93) (width 0.25) (layer B.Cu) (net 7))
 (segment (start 142.7 100.077) (end 140.448001 97.825001) (width 0.25) (layer F.Cu) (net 2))
 (segment (start 139.415001 97.825001) (end 137.54 95.95) (width 0.25) (layer F.Cu) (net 2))
 (segment (start 142.7 103) (end 142.7 100.077) (width 0.25) (layer F.Cu) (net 2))
 (segment (start 140.448001 97.825001) (end 139.415001 97.825001) (width 0.25) (layer F.Cu) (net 2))
 (segment (start 137.54 95.95) (end 137.54 94.825) (width 0.25) (layer F.Cu) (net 2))
 (via (at 137.5 93.199994) (size 0.8) (drill 0.4) (layers F.Cu B.Cu) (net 2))
 (segment (start 136.354999 64.724999) (end 136.354999 92.054993) (width 0.25) (layer B.Cu) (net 2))
 (segment (start 128.64 57.01) (end 136.354999 64.724999) (width 0.25) (layer B.Cu) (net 2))
 (segment (start 136.354999 92.054993) (end 137.5 93.199994) (width 0.25) (layer B.Cu) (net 2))
 (segment (start 137.54 94.825) (end 137.54 93.239994) (width 0.25) (layer F.Cu) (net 2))
 (segment (start 137.54 93.239994) (end 137.5 93.199994) (width 0.25) (layer F.Cu) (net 2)))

